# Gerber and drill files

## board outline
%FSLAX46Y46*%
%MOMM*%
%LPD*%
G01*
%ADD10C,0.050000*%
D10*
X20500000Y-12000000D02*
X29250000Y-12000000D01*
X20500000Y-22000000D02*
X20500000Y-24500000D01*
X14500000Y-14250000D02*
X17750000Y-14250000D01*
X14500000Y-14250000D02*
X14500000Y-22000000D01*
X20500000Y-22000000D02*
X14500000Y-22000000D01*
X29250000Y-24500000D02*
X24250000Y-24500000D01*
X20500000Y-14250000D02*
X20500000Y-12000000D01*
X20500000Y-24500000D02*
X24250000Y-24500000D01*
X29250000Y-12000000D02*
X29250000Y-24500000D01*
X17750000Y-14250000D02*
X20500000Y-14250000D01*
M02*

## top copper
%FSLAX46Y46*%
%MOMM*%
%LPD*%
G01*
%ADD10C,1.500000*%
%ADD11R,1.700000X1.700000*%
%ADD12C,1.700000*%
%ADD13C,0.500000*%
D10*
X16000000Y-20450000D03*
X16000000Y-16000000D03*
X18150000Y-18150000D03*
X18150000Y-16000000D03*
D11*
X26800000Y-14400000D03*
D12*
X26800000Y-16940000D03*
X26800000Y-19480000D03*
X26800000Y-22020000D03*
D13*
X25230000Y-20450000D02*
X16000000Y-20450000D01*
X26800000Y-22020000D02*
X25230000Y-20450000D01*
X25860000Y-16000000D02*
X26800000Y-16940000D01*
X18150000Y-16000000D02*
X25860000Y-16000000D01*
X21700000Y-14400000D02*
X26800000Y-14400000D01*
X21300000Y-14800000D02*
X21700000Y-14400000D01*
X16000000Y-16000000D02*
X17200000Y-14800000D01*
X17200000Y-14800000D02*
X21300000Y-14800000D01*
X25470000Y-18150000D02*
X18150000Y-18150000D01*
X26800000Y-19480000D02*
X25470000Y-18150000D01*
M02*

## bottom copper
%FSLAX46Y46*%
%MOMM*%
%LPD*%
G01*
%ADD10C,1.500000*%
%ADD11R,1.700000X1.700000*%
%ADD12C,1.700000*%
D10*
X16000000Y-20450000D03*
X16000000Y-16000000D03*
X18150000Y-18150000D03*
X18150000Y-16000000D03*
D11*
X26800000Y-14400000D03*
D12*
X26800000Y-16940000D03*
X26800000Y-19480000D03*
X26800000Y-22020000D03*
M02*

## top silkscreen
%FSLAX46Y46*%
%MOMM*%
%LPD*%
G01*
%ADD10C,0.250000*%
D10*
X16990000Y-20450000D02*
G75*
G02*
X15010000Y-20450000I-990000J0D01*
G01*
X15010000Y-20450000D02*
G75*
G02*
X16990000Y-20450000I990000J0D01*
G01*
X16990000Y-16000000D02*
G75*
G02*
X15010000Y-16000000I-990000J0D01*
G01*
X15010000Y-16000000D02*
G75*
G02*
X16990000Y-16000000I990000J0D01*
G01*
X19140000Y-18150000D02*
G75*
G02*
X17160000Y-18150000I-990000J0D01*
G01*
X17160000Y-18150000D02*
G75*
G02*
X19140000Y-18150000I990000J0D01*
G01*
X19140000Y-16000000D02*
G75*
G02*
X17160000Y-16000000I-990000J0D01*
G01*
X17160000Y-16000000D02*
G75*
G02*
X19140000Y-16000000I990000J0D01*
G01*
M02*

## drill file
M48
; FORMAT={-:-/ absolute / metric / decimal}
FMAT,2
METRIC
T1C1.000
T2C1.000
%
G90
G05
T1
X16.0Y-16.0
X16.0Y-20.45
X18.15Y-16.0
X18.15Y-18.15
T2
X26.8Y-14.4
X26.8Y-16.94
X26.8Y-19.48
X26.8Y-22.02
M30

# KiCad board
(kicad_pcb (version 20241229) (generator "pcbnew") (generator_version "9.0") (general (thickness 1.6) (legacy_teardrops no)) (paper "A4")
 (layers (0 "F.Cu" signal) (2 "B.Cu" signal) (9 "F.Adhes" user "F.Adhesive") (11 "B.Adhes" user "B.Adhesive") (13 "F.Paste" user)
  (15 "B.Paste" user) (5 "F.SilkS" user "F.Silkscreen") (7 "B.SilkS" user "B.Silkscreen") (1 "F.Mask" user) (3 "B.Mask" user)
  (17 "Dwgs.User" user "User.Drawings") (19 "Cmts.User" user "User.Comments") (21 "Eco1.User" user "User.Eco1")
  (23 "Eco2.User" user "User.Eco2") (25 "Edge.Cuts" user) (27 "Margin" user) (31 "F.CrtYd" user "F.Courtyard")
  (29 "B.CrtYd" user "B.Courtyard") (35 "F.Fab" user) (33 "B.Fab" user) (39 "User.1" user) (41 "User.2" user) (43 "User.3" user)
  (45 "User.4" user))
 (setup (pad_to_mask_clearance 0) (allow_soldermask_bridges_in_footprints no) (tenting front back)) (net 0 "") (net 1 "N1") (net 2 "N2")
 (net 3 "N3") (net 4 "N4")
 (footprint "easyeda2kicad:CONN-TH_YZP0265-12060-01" (layer "F.Cu") (at 16 20.45)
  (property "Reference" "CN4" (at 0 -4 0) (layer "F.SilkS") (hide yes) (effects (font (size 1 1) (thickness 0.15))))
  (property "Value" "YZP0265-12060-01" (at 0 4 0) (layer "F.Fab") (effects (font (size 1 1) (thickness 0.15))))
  (fp_circle (center 0 0) (end 0.99 0) (stroke (width 0.25) (type solid)) (fill no) (layer "F.SilkS"))
  (pad "1" thru_hole circle (at 0 0) (size 1.5 1.5) (drill 0.999998) (layers "*.Cu" "*.Mask") (remove_unused_layers no) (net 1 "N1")))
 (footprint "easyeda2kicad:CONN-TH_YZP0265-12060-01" (layer "F.Cu") (at 16 16)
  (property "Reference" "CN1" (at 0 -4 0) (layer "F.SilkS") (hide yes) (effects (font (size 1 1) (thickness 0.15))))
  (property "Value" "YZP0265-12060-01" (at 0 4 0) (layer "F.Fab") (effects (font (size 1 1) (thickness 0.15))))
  (fp_circle (center 0 0) (end 0.99 0) (stroke (width 0.25) (type solid)) (fill no) (layer "F.SilkS"))
  (pad "1" thru_hole circle (at 0 0) (size 1.5 1.5) (drill 0.999998) (layers "*.Cu" "*.Mask") (remove_unused_layers no) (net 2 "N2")))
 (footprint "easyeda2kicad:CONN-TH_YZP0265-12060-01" (layer "F.Cu") (at 18.15 18.15)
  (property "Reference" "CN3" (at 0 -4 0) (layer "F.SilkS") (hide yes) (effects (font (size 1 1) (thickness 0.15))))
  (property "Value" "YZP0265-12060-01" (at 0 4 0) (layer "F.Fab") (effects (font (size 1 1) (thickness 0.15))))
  (fp_circle (center 0 0) (end 0.99 0) (stroke (width 0.25) (type solid)) (fill no) (layer "F.SilkS"))
  (pad "1" thru_hole circle (at 0 0) (size 1.5 1.5) (drill 0.999998) (layers "*.Cu" "*.Mask") (remove_unused_layers no) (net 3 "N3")))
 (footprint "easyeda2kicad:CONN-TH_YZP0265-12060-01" (layer "F.Cu") (at 18.15 16)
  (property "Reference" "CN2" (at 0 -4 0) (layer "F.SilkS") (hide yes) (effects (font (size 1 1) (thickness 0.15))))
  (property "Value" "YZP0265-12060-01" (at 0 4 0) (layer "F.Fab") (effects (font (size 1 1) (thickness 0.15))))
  (fp_circle (center 0 0) (end 0.99 0) (stroke (width 0.25) (type solid)) (fill no) (layer "F.SilkS"))
  (pad "1" thru_hole circle (at 0 0) (size 1.5 1.5) (drill 0.999998) (layers "*.Cu" "*.Mask") (remove_unused_layers no) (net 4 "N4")))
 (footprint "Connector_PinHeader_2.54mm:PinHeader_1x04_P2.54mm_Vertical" (layer "B.Cu") (at 26.8 14.4 180)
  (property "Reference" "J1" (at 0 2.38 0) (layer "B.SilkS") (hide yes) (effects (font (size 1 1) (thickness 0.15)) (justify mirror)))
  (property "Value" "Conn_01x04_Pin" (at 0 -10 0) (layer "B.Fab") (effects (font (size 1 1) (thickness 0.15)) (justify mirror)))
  (pad "1" thru_hole rect (at 0 0 180) (size 1.7 1.7) (drill 1) (layers "*.Cu" "*.Mask") (remove_unused_layers no) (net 2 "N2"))
  (pad "2" thru_hole circle (at 0 -2.54 180) (size 1.7 1.7) (drill 1) (layers "*.Cu" "*.Mask") (remove_unused_layers no) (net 4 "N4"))
  (pad "3" thru_hole circle (at 0 -5.08 180) (size 1.7 1.7) (drill 1) (layers "*.Cu" "*.Mask") (remove_unused_layers no) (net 3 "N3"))
  (pad "4" thru_hole circle (at 0 -7.62 180) (size 1.7 1.7) (drill 1) (layers "*.Cu" "*.Mask") (remove_unused_layers no) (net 1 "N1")))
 (gr_line (start 20.5 12) (end 29.25 12) (stroke (width 0.05) (type default)) (layer "Edge.Cuts"))
 (gr_line (start 20.5 22) (end 20.5 24.5) (stroke (width 0.05) (type default)) (layer "Edge.Cuts"))
 (gr_line (start 14.5 14.25) (end 17.75 14.25) (stroke (width 0.05) (type default)) (layer "Edge.Cuts"))
 (gr_line (start 14.5 14.25) (end 14.5 22) (stroke (width 0.05) (type default)) (layer "Edge.Cuts"))
 (gr_line (start 20.5 22) (end 14.5 22) (stroke (width 0.05) (type default)) (layer "Edge.Cuts"))
 (gr_line (start 29.25 24.5) (end 24.25 24.5) (stroke (width 0.05) (type default)) (layer "Edge.Cuts"))
 (gr_line (start 20.5 14.25) (end 20.5 12) (stroke (width 0.05) (type default)) (layer "Edge.Cuts"))
 (gr_line (start 20.5 24.5) (end 24.25 24.5) (stroke (width 0.05) (type default)) (layer "Edge.Cuts"))
 (gr_line (start 29.25 12) (end 29.25 24.5) (stroke (width 0.05) (type default)) (layer "Edge.Cuts"))
 (gr_line (start 17.75 14.25) (end 20.5 14.25) (stroke (width 0.05) (type default)) (layer "Edge.Cuts"))
 (segment (start 25.23 20.45) (end 16 20.45) (width 0.5) (layer "F.Cu") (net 1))
 (segment (start 26.8 22.02) (end 25.23 20.45) (width 0.5) (layer "F.Cu") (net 1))
 (segment (start 25.86 16) (end 26.8 16.94) (width 0.5) (layer "F.Cu") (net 4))
 (segment (start 18.15 16) (end 25.86 16) (width 0.5) (layer "F.Cu") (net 4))
 (segment (start 21.7 14.4) (end 26.8 14.4) (width 0.5) (layer "F.Cu") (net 2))
 (segment (start 21.3 14.8) (end 21.7 14.4) (width 0.5) (layer "F.Cu") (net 2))
 (segment (start 16 16) (end 17.2 14.8) (width 0.5) (layer "F.Cu") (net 2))
 (segment (start 17.2 14.8) (end 21.3 14.8) (width 0.5) (layer "F.Cu") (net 2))
 (segment (start 25.47 18.15) (end 18.15 18.15) (width 0.5) (layer "F.Cu") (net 3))
 (segment (start 26.8 19.48) (end 25.47 18.15) (width 0.5) (layer "F.Cu") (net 3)))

